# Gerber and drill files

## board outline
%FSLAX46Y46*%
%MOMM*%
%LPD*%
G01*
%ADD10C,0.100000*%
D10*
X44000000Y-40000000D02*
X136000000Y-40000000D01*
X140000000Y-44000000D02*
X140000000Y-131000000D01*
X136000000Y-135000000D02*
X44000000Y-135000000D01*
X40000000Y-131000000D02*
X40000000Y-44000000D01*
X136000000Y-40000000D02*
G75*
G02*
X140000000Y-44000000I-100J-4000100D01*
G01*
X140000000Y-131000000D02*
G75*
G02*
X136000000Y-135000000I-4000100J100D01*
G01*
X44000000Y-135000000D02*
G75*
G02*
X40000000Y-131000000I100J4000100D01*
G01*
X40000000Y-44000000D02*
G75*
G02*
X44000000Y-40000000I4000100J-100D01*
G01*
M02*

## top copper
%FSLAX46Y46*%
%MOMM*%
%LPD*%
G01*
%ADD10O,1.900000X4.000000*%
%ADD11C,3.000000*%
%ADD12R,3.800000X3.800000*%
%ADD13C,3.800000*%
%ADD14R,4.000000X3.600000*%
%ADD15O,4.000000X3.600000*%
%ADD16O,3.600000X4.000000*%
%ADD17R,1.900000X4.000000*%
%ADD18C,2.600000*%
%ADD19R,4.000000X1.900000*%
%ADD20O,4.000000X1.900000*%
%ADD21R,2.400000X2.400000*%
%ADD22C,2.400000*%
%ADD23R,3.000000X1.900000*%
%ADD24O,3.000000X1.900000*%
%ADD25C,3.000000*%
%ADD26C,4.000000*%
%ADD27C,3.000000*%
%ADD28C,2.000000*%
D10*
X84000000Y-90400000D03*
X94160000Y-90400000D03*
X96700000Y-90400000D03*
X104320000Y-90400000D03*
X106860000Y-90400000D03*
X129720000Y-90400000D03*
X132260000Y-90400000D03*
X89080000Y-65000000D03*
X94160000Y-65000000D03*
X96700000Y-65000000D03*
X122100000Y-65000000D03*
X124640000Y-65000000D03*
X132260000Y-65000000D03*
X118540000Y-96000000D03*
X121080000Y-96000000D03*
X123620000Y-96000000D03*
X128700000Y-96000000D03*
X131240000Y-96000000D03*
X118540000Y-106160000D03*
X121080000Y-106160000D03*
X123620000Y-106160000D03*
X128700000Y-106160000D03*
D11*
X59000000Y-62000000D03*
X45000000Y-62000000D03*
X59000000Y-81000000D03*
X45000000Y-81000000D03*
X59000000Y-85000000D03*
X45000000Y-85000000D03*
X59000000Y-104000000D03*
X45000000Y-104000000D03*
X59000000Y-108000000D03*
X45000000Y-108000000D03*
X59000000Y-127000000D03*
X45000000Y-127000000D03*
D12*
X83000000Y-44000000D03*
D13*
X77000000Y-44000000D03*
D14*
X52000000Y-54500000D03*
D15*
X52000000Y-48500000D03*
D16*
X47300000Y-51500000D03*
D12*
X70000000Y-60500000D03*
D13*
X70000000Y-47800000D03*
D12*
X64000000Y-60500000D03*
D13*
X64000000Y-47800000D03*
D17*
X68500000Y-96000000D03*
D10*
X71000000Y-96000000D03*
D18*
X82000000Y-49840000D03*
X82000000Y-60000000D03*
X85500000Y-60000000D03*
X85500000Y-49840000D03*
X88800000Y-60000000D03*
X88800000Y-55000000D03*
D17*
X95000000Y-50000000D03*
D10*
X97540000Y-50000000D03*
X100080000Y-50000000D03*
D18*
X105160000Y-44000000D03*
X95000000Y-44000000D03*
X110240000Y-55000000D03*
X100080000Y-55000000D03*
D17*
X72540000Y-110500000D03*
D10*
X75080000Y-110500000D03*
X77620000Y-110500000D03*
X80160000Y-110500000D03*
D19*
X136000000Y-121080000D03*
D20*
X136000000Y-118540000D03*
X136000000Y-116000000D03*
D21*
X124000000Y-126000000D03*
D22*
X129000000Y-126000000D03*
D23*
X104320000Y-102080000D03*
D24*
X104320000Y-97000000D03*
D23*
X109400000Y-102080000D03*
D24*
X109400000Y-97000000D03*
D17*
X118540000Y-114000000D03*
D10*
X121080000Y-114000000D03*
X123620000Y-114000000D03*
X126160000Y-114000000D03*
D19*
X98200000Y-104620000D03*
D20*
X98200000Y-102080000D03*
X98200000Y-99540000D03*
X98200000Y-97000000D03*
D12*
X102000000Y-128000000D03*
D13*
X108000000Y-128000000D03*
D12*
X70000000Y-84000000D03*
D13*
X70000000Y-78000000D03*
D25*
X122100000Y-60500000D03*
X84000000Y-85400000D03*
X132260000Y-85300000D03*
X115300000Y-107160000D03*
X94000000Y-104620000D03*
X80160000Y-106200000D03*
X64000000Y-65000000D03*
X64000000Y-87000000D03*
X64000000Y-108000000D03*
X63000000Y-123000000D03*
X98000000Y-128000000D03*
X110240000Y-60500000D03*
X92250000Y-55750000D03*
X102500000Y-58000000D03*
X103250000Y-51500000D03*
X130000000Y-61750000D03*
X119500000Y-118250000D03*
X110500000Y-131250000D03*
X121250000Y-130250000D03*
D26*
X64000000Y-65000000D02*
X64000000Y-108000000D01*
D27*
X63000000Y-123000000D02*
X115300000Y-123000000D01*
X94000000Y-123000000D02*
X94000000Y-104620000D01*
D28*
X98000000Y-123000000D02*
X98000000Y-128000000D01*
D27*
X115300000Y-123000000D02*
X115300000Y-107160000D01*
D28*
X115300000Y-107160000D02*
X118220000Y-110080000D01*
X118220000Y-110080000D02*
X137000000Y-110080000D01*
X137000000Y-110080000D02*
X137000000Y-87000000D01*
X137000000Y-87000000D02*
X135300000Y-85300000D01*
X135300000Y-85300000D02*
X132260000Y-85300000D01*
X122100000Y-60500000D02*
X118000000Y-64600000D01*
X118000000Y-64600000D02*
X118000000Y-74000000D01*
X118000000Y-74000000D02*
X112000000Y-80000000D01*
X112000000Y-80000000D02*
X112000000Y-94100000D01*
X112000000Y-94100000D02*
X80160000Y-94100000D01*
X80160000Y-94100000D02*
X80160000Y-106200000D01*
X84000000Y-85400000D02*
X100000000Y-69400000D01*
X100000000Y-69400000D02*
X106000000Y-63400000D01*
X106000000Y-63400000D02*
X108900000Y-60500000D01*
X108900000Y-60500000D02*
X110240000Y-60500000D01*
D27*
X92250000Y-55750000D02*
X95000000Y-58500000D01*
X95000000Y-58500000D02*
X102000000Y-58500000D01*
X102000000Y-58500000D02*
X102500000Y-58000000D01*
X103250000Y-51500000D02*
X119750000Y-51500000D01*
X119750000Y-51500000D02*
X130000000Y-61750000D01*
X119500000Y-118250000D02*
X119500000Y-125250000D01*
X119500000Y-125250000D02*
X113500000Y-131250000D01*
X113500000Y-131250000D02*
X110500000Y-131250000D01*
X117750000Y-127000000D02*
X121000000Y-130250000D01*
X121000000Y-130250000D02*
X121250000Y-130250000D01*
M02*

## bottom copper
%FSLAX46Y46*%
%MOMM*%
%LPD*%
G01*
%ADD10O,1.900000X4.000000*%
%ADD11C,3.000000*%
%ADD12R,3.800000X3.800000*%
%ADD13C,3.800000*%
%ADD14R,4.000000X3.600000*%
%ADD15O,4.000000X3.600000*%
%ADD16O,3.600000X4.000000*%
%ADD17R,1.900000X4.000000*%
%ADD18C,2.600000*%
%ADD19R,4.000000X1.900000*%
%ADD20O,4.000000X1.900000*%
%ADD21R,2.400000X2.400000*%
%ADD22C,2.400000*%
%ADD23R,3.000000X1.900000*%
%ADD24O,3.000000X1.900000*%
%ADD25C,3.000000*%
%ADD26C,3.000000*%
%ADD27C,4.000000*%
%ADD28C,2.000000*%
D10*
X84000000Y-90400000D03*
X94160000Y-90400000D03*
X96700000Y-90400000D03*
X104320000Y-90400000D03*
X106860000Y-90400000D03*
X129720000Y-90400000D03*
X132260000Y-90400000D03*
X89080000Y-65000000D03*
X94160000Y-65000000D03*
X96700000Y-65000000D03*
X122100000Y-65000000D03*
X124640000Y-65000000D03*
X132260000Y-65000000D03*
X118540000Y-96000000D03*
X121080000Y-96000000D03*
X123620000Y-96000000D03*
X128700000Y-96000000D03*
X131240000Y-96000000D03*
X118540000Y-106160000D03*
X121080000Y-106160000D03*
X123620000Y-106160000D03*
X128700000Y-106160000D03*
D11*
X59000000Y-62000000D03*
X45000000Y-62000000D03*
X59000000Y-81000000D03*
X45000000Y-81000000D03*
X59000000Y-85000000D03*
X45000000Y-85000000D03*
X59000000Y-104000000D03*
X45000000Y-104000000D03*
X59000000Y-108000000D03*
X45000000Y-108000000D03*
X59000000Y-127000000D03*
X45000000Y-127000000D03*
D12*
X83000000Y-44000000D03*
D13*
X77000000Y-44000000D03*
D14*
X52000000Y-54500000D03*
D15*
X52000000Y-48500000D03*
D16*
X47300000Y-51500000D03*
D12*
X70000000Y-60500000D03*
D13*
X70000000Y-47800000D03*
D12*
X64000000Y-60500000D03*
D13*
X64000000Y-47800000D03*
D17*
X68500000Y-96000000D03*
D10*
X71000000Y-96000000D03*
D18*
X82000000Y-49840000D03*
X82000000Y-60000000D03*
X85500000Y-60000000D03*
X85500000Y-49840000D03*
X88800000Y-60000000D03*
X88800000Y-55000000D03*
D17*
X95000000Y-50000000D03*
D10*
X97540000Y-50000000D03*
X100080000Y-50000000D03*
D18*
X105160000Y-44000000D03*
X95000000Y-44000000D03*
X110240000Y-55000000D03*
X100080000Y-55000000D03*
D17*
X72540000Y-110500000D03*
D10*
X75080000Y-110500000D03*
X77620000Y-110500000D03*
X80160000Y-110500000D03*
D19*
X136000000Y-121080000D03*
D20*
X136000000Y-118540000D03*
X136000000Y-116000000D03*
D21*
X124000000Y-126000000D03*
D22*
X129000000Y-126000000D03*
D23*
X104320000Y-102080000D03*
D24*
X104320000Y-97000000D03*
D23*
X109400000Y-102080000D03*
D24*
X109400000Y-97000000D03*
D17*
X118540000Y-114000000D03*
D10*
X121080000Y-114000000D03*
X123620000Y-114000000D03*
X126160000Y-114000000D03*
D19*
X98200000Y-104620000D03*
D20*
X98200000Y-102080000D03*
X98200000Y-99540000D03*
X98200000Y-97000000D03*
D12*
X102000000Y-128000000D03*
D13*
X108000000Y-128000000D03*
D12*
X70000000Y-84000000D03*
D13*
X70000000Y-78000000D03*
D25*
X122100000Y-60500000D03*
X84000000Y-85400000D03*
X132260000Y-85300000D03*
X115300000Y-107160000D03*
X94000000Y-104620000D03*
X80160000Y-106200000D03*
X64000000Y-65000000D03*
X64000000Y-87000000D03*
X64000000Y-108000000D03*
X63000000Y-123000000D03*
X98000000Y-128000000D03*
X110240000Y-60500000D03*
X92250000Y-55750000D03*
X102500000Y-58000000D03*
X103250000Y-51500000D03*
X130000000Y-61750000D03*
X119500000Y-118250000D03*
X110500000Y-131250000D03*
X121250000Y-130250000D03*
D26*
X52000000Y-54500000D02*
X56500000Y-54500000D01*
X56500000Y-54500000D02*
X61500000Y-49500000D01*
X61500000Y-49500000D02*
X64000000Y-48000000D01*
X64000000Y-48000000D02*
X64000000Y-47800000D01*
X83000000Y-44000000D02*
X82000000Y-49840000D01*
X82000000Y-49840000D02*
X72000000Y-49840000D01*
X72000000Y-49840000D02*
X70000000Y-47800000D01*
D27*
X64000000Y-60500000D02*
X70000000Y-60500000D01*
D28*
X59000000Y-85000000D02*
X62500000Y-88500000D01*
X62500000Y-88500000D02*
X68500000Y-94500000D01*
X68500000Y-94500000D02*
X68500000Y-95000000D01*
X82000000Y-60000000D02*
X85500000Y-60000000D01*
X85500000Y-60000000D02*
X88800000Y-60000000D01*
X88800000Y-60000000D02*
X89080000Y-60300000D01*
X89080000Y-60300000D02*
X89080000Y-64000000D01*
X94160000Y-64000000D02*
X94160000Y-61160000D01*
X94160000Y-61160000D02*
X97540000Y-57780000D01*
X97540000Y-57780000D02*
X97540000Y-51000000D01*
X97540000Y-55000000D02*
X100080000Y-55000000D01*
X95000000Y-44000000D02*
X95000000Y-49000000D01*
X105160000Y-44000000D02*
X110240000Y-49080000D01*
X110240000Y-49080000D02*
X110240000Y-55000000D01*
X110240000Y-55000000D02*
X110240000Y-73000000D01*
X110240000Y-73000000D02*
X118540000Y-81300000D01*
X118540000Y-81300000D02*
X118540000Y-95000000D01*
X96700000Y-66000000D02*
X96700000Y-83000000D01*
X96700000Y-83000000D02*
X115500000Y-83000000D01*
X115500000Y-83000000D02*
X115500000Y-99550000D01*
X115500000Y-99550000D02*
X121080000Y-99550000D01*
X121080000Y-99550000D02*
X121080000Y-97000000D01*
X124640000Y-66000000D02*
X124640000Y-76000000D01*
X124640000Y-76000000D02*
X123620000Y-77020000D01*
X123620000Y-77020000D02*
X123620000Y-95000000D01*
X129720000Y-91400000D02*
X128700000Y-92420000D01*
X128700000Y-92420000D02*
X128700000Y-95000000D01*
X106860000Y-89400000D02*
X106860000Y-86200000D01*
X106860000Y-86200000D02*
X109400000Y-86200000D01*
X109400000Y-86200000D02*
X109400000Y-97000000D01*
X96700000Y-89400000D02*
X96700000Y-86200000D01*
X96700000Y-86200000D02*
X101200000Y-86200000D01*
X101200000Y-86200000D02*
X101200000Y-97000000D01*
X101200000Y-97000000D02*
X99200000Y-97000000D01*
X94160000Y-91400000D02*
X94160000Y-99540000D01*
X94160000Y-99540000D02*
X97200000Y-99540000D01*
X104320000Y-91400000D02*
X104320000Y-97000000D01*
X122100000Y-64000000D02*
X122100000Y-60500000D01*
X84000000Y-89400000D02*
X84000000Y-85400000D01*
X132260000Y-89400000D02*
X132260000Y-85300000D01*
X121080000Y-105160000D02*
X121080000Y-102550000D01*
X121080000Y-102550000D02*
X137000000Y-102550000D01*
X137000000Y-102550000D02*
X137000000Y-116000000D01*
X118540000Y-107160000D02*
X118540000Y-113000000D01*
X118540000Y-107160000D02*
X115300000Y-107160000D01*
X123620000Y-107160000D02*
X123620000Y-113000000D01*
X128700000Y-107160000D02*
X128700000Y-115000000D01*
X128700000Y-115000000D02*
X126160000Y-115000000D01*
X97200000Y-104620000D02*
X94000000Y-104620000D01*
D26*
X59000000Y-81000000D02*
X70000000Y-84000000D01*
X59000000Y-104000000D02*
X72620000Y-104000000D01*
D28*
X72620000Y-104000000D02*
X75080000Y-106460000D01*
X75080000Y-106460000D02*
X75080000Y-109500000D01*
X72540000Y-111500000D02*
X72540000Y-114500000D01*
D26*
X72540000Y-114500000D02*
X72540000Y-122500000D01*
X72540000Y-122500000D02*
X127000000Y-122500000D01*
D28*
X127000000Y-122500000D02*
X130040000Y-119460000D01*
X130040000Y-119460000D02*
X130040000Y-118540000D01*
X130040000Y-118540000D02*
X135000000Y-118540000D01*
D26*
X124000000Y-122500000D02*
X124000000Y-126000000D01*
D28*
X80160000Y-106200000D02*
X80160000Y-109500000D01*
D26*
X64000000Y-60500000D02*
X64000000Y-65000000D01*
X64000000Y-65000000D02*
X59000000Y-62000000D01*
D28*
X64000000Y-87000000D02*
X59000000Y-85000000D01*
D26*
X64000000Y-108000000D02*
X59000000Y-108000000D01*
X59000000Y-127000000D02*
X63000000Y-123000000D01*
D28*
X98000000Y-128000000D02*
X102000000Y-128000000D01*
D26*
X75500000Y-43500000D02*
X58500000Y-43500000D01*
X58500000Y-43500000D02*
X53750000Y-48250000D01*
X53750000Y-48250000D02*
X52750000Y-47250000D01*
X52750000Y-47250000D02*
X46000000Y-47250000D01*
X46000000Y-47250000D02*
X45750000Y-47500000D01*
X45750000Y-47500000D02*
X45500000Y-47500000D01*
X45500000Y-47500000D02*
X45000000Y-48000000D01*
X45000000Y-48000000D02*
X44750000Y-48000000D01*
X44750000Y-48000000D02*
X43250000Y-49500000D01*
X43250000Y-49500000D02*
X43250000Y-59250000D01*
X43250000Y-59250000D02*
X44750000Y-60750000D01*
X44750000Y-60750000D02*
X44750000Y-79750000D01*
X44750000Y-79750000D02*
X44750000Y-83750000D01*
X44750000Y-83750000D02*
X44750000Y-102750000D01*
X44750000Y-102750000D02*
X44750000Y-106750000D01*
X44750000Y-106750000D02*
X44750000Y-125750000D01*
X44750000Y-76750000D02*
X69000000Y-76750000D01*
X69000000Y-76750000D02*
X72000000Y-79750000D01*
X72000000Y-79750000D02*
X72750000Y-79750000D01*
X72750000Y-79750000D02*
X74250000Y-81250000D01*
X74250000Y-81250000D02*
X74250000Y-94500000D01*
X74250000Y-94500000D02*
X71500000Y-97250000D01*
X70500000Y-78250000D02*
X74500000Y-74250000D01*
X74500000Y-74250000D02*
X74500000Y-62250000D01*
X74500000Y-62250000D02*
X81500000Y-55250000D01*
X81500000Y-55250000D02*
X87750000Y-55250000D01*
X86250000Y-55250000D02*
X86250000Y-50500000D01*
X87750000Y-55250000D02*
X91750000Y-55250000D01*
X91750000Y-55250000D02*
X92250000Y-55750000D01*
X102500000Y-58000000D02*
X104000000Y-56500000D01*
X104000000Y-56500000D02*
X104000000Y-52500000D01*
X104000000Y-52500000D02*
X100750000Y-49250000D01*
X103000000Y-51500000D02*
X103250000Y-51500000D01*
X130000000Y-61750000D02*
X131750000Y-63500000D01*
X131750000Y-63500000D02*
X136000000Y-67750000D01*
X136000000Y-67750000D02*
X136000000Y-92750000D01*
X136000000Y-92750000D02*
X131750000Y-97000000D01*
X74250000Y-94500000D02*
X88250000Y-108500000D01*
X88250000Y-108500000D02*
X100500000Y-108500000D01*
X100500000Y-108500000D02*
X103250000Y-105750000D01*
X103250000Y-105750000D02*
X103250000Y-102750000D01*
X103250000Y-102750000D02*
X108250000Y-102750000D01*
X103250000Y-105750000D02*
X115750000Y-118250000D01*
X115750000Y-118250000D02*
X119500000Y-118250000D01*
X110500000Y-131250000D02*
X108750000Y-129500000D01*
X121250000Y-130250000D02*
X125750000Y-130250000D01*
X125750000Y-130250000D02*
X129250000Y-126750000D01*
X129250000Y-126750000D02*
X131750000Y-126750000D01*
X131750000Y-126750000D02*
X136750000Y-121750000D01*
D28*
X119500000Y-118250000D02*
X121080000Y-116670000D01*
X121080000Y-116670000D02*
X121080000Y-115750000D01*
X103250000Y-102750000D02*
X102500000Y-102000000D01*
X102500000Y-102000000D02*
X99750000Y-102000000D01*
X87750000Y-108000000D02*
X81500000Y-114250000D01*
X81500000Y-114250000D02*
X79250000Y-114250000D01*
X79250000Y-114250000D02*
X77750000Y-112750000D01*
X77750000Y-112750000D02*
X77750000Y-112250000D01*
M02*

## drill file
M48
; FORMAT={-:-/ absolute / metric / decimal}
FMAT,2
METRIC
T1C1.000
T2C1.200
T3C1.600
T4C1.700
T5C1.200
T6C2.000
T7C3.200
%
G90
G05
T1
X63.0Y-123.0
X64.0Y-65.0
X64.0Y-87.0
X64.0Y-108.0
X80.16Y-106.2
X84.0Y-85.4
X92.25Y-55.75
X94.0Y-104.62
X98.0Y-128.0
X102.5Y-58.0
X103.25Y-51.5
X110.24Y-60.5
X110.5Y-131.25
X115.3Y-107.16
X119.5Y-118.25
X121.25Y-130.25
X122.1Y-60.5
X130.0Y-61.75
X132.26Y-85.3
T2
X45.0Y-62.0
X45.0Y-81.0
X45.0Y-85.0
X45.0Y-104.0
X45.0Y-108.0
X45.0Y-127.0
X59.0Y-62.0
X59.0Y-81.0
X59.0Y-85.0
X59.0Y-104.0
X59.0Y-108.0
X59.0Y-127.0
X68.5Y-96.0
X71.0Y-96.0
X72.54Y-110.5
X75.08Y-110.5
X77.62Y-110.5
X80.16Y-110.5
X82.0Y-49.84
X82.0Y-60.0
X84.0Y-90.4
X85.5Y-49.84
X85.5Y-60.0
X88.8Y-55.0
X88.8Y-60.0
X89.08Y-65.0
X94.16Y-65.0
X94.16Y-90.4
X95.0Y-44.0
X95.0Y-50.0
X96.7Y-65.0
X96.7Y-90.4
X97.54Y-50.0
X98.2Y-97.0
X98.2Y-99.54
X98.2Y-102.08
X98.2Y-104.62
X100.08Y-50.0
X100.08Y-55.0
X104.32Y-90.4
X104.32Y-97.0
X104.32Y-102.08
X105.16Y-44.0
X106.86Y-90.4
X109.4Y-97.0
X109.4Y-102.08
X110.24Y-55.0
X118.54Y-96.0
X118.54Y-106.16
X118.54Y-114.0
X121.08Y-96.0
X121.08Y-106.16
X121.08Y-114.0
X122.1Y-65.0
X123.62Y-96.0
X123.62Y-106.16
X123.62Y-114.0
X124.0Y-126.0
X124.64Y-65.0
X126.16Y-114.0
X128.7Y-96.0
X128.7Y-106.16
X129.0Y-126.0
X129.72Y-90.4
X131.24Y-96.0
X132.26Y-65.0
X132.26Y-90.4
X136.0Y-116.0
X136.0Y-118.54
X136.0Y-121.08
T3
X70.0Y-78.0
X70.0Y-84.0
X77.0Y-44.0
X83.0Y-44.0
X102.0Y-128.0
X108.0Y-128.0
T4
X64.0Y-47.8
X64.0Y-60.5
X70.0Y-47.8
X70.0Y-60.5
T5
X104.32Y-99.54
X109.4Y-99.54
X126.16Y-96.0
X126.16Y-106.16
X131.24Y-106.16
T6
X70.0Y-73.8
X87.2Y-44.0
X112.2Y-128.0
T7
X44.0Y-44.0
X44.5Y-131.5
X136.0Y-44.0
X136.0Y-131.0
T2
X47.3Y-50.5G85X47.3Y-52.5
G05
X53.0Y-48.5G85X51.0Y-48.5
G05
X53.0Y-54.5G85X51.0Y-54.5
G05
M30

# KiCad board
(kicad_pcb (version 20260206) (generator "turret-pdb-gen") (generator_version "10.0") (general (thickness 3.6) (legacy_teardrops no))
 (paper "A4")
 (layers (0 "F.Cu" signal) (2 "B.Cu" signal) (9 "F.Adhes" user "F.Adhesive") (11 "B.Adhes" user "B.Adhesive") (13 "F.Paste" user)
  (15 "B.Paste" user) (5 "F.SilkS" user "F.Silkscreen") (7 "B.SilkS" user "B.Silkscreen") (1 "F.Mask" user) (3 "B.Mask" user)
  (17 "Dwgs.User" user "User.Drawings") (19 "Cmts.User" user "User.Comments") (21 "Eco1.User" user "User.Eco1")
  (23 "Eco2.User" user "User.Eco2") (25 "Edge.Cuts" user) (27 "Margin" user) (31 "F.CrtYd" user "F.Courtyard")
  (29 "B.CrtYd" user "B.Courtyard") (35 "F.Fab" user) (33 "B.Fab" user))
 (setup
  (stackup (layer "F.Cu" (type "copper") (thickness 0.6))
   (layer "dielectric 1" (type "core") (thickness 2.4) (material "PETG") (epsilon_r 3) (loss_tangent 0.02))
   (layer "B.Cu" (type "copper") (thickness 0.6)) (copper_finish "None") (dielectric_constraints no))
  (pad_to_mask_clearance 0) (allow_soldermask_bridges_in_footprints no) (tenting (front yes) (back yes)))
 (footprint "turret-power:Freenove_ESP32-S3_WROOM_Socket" (layer "F.Cu") (at 84 90.4)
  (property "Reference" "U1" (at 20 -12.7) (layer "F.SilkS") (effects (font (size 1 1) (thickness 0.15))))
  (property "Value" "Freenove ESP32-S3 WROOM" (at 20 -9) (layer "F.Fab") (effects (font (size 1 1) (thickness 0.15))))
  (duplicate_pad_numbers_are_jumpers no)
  (pad "L1" thru_hole oval (at 0 0) (size 1.9 4) (drill 1.2) (layers "*.Cu" "B.Mask") (zone_connect 0) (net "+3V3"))
  (pad "L5" thru_hole oval (at 10.16 0) (size 1.9 4) (drill 1.2) (layers "*.Cu" "B.Mask") (zone_connect 0) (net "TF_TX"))
  (pad "L6" thru_hole oval (at 12.7 0) (size 1.9 4) (drill 1.2) (layers "*.Cu" "B.Mask") (zone_connect 0) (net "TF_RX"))
  (pad "L9" thru_hole oval (at 20.32 0) (size 1.9 4) (drill 1.2) (layers "*.Cu" "B.Mask") (zone_connect 0) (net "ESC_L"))
  (pad "L10" thru_hole oval (at 22.86 0) (size 1.9 4) (drill 1.2) (layers "*.Cu" "B.Mask") (zone_connect 0) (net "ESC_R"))
  (pad "L19" thru_hole oval (at 45.72 0) (size 1.9 4) (drill 1.2) (layers "*.Cu" "B.Mask") (zone_connect 0) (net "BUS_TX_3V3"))
  (pad "L20" thru_hole oval (at 48.26 0) (size 1.9 4) (drill 1.2) (layers "*.Cu" "B.Mask") (zone_connect 0) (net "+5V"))
  (pad "R3" thru_hole oval (at 5.08 -25.4) (size 1.9 4) (drill 1.2) (layers "*.Cu" "B.Mask") (zone_connect 0) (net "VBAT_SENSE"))
  (pad "R5" thru_hole oval (at 10.16 -25.4) (size 1.9 4) (drill 1.2) (layers "*.Cu" "B.Mask") (zone_connect 0) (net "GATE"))
  (pad "R6" thru_hole oval (at 12.7 -25.4) (size 1.9 4) (drill 1.2) (layers "*.Cu" "B.Mask") (zone_connect 0) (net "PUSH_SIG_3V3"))
  (pad "R16" thru_hole oval (at 38.1 -25.4) (size 1.9 4) (drill 1.2) (layers "*.Cu" "B.Mask") (zone_connect 0) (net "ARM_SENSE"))
  (pad "R17" thru_hole oval (at 40.64 -25.4) (size 1.9 4) (drill 1.2) (layers "*.Cu" "B.Mask") (zone_connect 0) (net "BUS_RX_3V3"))
  (pad "R20" thru_hole oval (at 48.26 -25.4) (size 1.9 4) (drill 1.2) (layers "*.Cu" "B.Mask") (zone_connect 0) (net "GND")))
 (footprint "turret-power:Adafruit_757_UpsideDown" (layer "F.Cu") (at 118.54 96)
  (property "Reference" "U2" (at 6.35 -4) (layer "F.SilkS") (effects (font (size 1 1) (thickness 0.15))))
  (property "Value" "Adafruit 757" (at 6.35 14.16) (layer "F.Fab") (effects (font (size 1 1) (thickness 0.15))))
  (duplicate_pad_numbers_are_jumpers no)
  (pad "LV" thru_hole oval (at 0 0) (size 1.9 4) (drill 1.2) (layers "*.Cu" "B.Mask") (zone_connect 0) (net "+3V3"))
  (pad "A1" thru_hole oval (at 2.54 0) (size 1.9 4) (drill 1.2) (layers "*.Cu" "B.Mask") (zone_connect 0) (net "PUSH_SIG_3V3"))
  (pad "A2" thru_hole oval (at 5.08 0) (size 1.9 4) (drill 1.2) (layers "*.Cu" "B.Mask") (zone_connect 0) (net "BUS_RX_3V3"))
  (pad "" np_thru_hole circle (at 7.62 0) (size 1.2 1.2) (drill 1.2) (layers "*.Cu" "*.Mask"))
  (pad "A4" thru_hole oval (at 10.16 0) (size 1.9 4) (drill 1.2) (layers "*.Cu" "B.Mask") (zone_connect 0) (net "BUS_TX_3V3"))
  (pad "GND_LV" thru_hole oval (at 12.7 0) (size 1.9 4) (drill 1.2) (layers "*.Cu" "B.Mask") (zone_connect 0) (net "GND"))
  (pad "HV" thru_hole oval (at 0 10.16) (size 1.9 4) (drill 1.2) (layers "*.Cu" "B.Mask") (zone_connect 0) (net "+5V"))
  (pad "B1" thru_hole oval (at 2.54 10.16) (size 1.9 4) (drill 1.2) (layers "*.Cu" "B.Mask") (zone_connect 0) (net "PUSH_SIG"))
  (pad "B2" thru_hole oval (at 5.08 10.16) (size 1.9 4) (drill 1.2) (layers "*.Cu" "B.Mask") (zone_connect 0) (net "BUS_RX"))
  (pad "" np_thru_hole circle (at 7.62 10.16) (size 1.2 1.2) (drill 1.2) (layers "*.Cu" "*.Mask"))
  (pad "B4" thru_hole oval (at 10.16 10.16) (size 1.9 4) (drill 1.2) (layers "*.Cu" "B.Mask") (zone_connect 0) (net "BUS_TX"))
  (pad "" np_thru_hole circle (at 12.7 10.16) (size 1.2 1.2) (drill 1.2) (layers "*.Cu" "*.Mask")))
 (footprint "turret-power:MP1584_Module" (layer "F.Cu") (at 59 62 270)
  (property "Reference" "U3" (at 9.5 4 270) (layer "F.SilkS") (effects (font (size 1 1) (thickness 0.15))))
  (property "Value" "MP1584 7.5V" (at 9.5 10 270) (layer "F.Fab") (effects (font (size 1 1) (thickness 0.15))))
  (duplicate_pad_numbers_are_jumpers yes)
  (pad "VIN" thru_hole circle (at 0 0 270) (size 3 3) (drill 1.2) (layers "*.Cu" "*.Mask") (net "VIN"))
  (pad "GND" thru_hole circle (at 0 14 270) (size 3 3) (drill 1.2) (layers "*.Cu" "*.Mask") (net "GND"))
  (pad "VOUT" thru_hole circle (at 19 0 270) (size 3 3) (drill 1.2) (layers "*.Cu" "*.Mask") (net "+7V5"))
  (pad "GND" thru_hole circle (at 19 14 270) (size 3 3) (drill 1.2) (layers "*.Cu" "*.Mask") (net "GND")))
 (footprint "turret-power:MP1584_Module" (layer "F.Cu") (at 59 85 270)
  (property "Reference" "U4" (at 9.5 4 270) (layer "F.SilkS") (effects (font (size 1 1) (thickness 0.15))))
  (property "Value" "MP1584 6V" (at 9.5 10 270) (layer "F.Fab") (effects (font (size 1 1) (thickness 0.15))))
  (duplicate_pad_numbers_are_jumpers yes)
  (pad "VIN" thru_hole circle (at 0 0 270) (size 3 3) (drill 1.2) (layers "*.Cu" "*.Mask") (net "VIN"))
  (pad "GND" thru_hole circle (at 0 14 270) (size 3 3) (drill 1.2) (layers "*.Cu" "*.Mask") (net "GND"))
  (pad "VOUT" thru_hole circle (at 19 0 270) (size 3 3) (drill 1.2) (layers "*.Cu" "*.Mask") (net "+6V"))
  (pad "GND" thru_hole circle (at 19 14 270) (size 3 3) (drill 1.2) (layers "*.Cu" "*.Mask") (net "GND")))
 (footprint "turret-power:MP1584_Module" (layer "F.Cu") (at 59 108 270)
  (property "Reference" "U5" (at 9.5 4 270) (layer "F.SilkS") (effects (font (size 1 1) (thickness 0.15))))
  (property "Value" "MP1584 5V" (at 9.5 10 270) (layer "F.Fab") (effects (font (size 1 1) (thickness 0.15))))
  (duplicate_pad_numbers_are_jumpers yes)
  (pad "VIN" thru_hole circle (at 0 0 270) (size 3 3) (drill 1.2) (layers "*.Cu" "*.Mask") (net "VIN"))
  (pad "GND" thru_hole circle (at 0 14 270) (size 3 3) (drill 1.2) (layers "*.Cu" "*.Mask") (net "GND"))
  (pad "VOUT" thru_hole circle (at 19 0 270) (size 3 3) (drill 1.2) (layers "*.Cu" "*.Mask") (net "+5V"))
  (pad "GND" thru_hole circle (at 19 14 270) (size 3 3) (drill 1.2) (layers "*.Cu" "*.Mask") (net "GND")))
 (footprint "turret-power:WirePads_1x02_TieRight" (layer "F.Cu") (at 83 44 180)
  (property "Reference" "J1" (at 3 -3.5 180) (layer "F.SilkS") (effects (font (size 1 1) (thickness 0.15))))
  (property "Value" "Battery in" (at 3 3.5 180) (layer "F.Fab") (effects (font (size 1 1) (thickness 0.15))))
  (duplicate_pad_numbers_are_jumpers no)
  (pad "1" thru_hole rect (at 0 0 180) (size 3.8 3.8) (drill 1.6) (layers "*.Cu" "*.Mask") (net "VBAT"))
  (pad "2" thru_hole circle (at 6 0 180) (size 3.8 3.8) (drill 1.6) (layers "*.Cu" "*.Mask") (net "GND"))
  (pad "" np_thru_hole circle (at -4.2 0) (size 2 2) (drill 2) (layers "*.Cu" "*.Mask")))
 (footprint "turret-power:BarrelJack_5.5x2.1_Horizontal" (layer "F.Cu") (at 52 54.5 270)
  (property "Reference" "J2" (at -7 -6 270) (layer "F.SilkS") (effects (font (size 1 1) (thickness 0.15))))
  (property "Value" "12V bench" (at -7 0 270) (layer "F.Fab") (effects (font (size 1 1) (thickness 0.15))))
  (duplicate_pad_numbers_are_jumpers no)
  (pad "1" thru_hole rect (at 0 0 270) (size 3.6 4) (drill oval 1.2 3.2) (layers "*.Cu" "B.Mask") (zone_connect 0) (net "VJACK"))
  (pad "2" thru_hole oval (at -6 0 270) (size 3.6 4) (drill oval 1.2 3.2) (layers "*.Cu" "B.Mask") (zone_connect 0) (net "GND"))
  (pad "3" thru_hole oval (at -3 4.7 270) (size 4 3.6) (drill oval 3.2 1.2) (layers "*.Cu" "B.Mask") (zone_connect 0)
   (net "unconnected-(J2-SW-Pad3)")))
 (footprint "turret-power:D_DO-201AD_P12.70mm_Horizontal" (layer "F.Cu") (at 70 60.5 90)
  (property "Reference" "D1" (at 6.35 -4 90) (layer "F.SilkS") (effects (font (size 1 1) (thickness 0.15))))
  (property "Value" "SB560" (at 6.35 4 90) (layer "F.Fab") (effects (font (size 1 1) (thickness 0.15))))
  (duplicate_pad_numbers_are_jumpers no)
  (pad "1" thru_hole rect (at 0 0 90) (size 3.8 3.8) (drill 1.7) (layers "*.Cu" "*.Mask") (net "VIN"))
  (pad "2" thru_hole circle (at 12.7 0 90) (size 3.8 3.8) (drill 1.7) (layers "*.Cu" "*.Mask") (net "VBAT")))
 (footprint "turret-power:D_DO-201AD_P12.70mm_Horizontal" (layer "F.Cu") (at 64 60.5 90)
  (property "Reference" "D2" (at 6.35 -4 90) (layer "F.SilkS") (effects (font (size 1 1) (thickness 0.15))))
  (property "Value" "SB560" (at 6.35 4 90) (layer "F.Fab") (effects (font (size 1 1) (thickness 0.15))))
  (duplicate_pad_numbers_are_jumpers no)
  (pad "1" thru_hole rect (at 0 0 90) (size 3.8 3.8) (drill 1.7) (layers "*.Cu" "*.Mask") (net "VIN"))
  (pad "2" thru_hole circle (at 12.7 0 90) (size 3.8 3.8) (drill 1.7) (layers "*.Cu" "*.Mask") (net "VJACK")))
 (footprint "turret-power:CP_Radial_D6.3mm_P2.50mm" (layer "F.Cu") (at 68.5 96)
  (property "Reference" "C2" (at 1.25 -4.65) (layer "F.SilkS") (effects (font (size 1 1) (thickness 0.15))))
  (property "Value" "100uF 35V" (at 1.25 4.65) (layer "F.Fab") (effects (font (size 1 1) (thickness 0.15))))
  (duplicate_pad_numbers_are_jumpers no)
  (pad "1" thru_hole rect (at 0 0) (size 1.9 4) (drill 1.2) (layers "*.Cu" "B.Mask") (zone_connect 0) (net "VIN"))
  (pad "2" thru_hole oval (at 2.5 0) (size 1.9 4) (drill 1.2) (layers "*.Cu" "B.Mask") (zone_connect 0) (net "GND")))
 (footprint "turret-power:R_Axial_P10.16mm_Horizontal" (layer "F.Cu") (at 82 49.84 270)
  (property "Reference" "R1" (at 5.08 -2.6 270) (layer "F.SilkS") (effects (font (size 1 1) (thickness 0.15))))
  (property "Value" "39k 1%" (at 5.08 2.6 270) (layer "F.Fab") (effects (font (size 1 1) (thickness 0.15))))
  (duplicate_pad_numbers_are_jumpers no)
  (pad "1" thru_hole circle (at 0 0 270) (size 2.6 2.6) (drill 1.2) (layers "*.Cu" "*.Mask") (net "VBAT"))
  (pad "2" thru_hole circle (at 10.16 0 270) (size 2.6 2.6) (drill 1.2) (layers "*.Cu" "*.Mask") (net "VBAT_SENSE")))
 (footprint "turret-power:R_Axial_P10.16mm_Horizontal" (layer "F.Cu") (at 85.5 60 90)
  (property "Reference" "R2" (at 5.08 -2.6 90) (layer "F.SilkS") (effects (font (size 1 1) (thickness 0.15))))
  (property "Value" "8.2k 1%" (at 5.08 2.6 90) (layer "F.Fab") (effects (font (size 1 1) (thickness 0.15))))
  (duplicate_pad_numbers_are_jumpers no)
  (pad "1" thru_hole circle (at 0 0 90) (size 2.6 2.6) (drill 1.2) (layers "*.Cu" "*.Mask") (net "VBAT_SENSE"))
  (pad "2" thru_hole circle (at 10.16 0 90) (size 2.6 2.6) (drill 1.2) (layers "*.Cu" "*.Mask") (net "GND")))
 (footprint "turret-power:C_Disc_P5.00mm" (layer "F.Cu") (at 88.8 60 90)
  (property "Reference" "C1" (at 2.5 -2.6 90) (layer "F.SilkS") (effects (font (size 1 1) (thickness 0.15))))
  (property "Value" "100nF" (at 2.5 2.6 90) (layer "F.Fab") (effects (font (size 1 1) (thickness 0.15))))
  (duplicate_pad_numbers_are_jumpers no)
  (pad "1" thru_hole circle (at 0 0 90) (size 2.6 2.6) (drill 1.2) (layers "*.Cu" "*.Mask") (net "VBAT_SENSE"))
  (pad "2" thru_hole circle (at 5 0 90) (size 2.6 2.6) (drill 1.2) (layers "*.Cu" "*.Mask") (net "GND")))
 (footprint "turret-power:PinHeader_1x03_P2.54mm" (layer "F.Cu") (at 95 50)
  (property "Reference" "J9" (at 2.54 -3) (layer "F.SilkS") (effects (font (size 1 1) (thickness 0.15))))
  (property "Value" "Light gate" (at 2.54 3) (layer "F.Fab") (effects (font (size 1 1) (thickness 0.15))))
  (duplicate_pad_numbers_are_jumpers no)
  (pad "1" thru_hole rect (at 0 0) (size 1.9 4) (drill 1.2) (layers "*.Cu" "B.Mask") (zone_connect 0) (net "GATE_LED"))
  (pad "2" thru_hole oval (at 2.54 0) (size 1.9 4) (drill 1.2) (layers "*.Cu" "B.Mask") (zone_connect 0) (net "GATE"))
  (pad "3" thru_hole oval (at 5.08 0) (size 1.9 4) (drill 1.2) (layers "*.Cu" "B.Mask") (zone_connect 0) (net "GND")))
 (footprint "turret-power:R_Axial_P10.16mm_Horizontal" (layer "F.Cu") (at 105.16 44 180)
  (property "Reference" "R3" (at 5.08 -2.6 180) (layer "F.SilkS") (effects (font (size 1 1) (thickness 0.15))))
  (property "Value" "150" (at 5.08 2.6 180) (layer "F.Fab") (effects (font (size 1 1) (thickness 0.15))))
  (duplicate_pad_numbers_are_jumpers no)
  (pad "1" thru_hole circle (at 0 0 180) (size 2.6 2.6) (drill 1.2) (layers "*.Cu" "*.Mask") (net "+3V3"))
  (pad "2" thru_hole circle (at 10.16 0 180) (size 2.6 2.6) (drill 1.2) (layers "*.Cu" "*.Mask") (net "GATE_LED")))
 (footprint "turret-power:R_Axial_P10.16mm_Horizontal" (layer "F.Cu") (at 110.24 55 180)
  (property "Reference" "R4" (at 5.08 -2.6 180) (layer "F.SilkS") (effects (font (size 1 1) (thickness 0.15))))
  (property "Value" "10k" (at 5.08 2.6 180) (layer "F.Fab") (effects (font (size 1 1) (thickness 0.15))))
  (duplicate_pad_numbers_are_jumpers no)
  (pad "1" thru_hole circle (at 0 0 180) (size 2.6 2.6) (drill 1.2) (layers "*.Cu" "*.Mask") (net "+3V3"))
  (pad "2" thru_hole circle (at 10.16 0 180) (size 2.6 2.6) (drill 1.2) (layers "*.Cu" "*.Mask") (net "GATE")))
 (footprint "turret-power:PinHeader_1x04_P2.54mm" (layer "F.Cu") (at 72.54 110.5)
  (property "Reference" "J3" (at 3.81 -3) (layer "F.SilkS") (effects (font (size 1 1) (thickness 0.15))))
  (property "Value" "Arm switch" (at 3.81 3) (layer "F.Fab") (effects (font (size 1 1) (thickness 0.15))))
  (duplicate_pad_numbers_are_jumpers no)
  (pad "1" thru_hole rect (at 0 0) (size 1.9 4) (drill 1.2) (layers "*.Cu" "B.Mask") (zone_connect 0) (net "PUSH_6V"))
  (pad "2" thru_hole oval (at 2.54 0) (size 1.9 4) (drill 1.2) (layers "*.Cu" "B.Mask") (zone_connect 0) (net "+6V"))
  (pad "3" thru_hole oval (at 5.08 0) (size 1.9 4) (drill 1.2) (layers "*.Cu" "B.Mask") (zone_connect 0) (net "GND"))
  (pad "4" thru_hole oval (at 7.62 0) (size 1.9 4) (drill 1.2) (layers "*.Cu" "B.Mask") (zone_connect 0) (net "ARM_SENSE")))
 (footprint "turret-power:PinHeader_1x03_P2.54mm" (layer "F.Cu") (at 136 121.08 90)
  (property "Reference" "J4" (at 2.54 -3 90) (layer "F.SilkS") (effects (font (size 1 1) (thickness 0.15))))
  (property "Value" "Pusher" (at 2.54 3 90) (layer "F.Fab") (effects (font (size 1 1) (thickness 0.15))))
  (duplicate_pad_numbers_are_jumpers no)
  (pad "1" thru_hole rect (at 0 0 90) (size 1.9 4) (drill 1.2) (layers "*.Cu" "B.Mask") (zone_connect 0) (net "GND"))
  (pad "2" thru_hole oval (at 2.54 0 90) (size 1.9 4) (drill 1.2) (layers "*.Cu" "B.Mask") (zone_connect 0) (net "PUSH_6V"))
  (pad "3" thru_hole oval (at 5.08 0 90) (size 1.9 4) (drill 1.2) (layers "*.Cu" "B.Mask") (zone_connect 0) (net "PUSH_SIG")))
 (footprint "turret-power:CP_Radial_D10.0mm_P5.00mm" (layer "F.Cu") (at 124 126)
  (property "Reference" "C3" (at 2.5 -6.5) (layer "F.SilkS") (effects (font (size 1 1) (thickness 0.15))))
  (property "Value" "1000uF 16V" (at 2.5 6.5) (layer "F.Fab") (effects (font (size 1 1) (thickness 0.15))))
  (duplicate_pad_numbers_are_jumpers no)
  (pad "1" thru_hole rect (at 0 0) (size 2.4 2.4) (drill 1.2) (layers "*.Cu" "B.Mask") (zone_connect 0) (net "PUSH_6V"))
  (pad "2" thru_hole circle (at 5 0) (size 2.4 2.4) (drill 1.2) (layers "*.Cu" "B.Mask") (zone_connect 0) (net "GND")))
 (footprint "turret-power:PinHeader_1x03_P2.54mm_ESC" (layer "F.Cu") (at 104.32 102.08 90)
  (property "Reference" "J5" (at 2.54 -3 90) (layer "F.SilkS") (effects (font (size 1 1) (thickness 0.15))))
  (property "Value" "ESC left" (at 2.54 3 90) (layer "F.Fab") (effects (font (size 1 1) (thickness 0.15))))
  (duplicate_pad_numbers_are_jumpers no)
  (pad "1" thru_hole rect (at 0 0 90) (size 1.9 3) (drill 1.2) (layers "*.Cu" "B.Mask") (zone_connect 0) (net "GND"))
  (pad "" np_thru_hole circle (at 2.54 0) (size 1.2 1.2) (drill 1.2) (layers "*.Cu" "*.Mask"))
  (pad "3" thru_hole oval (at 5.08 0 90) (size 1.9 3) (drill 1.2) (layers "*.Cu" "B.Mask") (zone_connect 0) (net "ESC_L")))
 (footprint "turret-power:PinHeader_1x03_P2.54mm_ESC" (layer "F.Cu") (at 109.4 102.08 90)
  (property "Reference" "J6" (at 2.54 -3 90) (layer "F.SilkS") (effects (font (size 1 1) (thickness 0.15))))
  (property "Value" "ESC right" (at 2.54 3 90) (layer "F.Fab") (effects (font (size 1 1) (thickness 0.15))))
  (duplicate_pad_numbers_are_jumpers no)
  (pad "1" thru_hole rect (at 0 0 90) (size 1.9 3) (drill 1.2) (layers "*.Cu" "B.Mask") (zone_connect 0) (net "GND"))
  (pad "" np_thru_hole circle (at 2.54 0) (size 1.2 1.2) (drill 1.2) (layers "*.Cu" "*.Mask"))
  (pad "3" thru_hole oval (at 5.08 0 90) (size 1.9 3) (drill 1.2) (layers "*.Cu" "B.Mask") (zone_connect 0) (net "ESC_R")))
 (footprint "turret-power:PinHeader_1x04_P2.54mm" (layer "F.Cu") (at 118.54 114)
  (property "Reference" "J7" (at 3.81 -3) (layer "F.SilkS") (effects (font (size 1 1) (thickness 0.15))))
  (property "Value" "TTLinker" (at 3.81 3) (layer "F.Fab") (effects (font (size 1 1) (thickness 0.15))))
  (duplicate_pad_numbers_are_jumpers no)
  (pad "1" thru_hole rect (at 0 0) (size 1.9 4) (drill 1.2) (layers "*.Cu" "B.Mask") (zone_connect 0) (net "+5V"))
  (pad "2" thru_hole oval (at 2.54 0) (size 1.9 4) (drill 1.2) (layers "*.Cu" "B.Mask") (zone_connect 0) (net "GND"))
  (pad "3" thru_hole oval (at 5.08 0) (size 1.9 4) (drill 1.2) (layers "*.Cu" "B.Mask") (zone_connect 0) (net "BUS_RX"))
  (pad "4" thru_hole oval (at 7.62 0) (size 1.9 4) (drill 1.2) (layers "*.Cu" "B.Mask") (zone_connect 0) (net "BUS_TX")))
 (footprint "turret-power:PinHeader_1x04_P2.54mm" (layer "F.Cu") (at 98.2 104.62 90)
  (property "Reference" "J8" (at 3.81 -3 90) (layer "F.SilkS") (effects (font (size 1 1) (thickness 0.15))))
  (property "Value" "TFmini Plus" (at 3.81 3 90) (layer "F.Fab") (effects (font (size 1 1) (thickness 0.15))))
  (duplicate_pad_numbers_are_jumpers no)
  (pad "1" thru_hole rect (at 0 0 90) (size 1.9 4) (drill 1.2) (layers "*.Cu" "B.Mask") (zone_connect 0) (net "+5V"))
  (pad "2" thru_hole oval (at 2.54 0 90) (size 1.9 4) (drill 1.2) (layers "*.Cu" "B.Mask") (zone_connect 0) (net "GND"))
  (pad "3" thru_hole oval (at 5.08 0 90) (size 1.9 4) (drill 1.2) (layers "*.Cu" "B.Mask") (zone_connect 0) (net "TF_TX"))
  (pad "4" thru_hole oval (at 7.62 0 90) (size 1.9 4) (drill 1.2) (layers "*.Cu" "B.Mask") (zone_connect 0) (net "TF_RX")))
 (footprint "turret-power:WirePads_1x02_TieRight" (layer "F.Cu") (at 102 128)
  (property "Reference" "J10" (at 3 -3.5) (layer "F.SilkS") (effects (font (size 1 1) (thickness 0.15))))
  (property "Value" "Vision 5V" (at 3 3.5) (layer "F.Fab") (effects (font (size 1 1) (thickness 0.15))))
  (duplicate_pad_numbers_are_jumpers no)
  (pad "1" thru_hole rect (at 0 0) (size 3.8 3.8) (drill 1.6) (layers "*.Cu" "*.Mask") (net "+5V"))
  (pad "2" thru_hole circle (at 6 0) (size 3.8 3.8) (drill 1.6) (layers "*.Cu" "*.Mask") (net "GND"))
  (pad "" np_thru_hole circle (at 10.2 0) (size 2 2) (drill 2) (layers "*.Cu" "*.Mask")))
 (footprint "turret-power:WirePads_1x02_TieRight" (layer "F.Cu") (at 70 84 90)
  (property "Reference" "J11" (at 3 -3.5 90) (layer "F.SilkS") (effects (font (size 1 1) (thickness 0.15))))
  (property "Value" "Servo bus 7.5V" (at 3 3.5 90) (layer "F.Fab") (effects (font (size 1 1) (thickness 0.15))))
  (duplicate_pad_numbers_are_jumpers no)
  (pad "1" thru_hole rect (at 0 0 90) (size 3.8 3.8) (drill 1.6) (layers "*.Cu" "*.Mask") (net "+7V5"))
  (pad "2" thru_hole circle (at 6 0 90) (size 3.8 3.8) (drill 1.6) (layers "*.Cu" "*.Mask") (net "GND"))
  (pad "" np_thru_hole circle (at 10.2 0) (size 2 2) (drill 2) (layers "*.Cu" "*.Mask")))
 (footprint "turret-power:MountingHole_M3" (layer "F.Cu") (at 44 44)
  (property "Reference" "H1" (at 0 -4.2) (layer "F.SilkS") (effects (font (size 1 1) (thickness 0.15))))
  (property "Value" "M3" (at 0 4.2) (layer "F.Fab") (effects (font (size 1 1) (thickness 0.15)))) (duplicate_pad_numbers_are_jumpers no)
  (pad "" np_thru_hole circle (at 0 0) (size 3.2 3.2) (drill 3.2) (layers "*.Cu" "*.Mask")))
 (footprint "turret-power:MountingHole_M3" (layer "F.Cu") (at 136 44)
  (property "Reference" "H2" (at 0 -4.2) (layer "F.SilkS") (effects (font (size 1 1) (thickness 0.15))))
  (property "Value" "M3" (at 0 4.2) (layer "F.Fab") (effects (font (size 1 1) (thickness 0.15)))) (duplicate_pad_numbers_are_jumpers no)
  (pad "" np_thru_hole circle (at 0 0) (size 3.2 3.2) (drill 3.2) (layers "*.Cu" "*.Mask")))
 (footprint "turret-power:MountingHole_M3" (layer "F.Cu") (at 44.5 131.5)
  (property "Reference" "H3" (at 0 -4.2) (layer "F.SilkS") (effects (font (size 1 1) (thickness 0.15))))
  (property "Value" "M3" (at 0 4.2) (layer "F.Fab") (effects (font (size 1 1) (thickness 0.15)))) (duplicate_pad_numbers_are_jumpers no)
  (pad "" np_thru_hole circle (at 0 0) (size 3.2 3.2) (drill 3.2) (layers "*.Cu" "*.Mask")))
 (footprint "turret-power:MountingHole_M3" (layer "F.Cu") (at 136 131)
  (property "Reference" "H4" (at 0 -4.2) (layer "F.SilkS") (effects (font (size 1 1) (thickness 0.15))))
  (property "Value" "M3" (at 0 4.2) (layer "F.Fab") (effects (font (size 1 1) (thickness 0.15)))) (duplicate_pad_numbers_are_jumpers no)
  (pad "" np_thru_hole circle (at 0 0) (size 3.2 3.2) (drill 3.2) (layers "*.Cu" "*.Mask")))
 (gr_line (start 44 40) (end 136 40) (stroke (width 0.1) (type default)) (layer "Edge.Cuts"))
 (gr_line (start 140 44) (end 140 131) (stroke (width 0.1) (type default)) (layer "Edge.Cuts"))
 (gr_line (start 136 135) (end 44 135) (stroke (width 0.1) (type default)) (layer "Edge.Cuts"))
 (gr_line (start 40 131) (end 40 44) (stroke (width 0.1) (type default)) (layer "Edge.Cuts"))
 (gr_arc (start 136 40) (mid 138.8284 41.1716) (end 140 44) (stroke (width 0.1) (type default)) (layer "Edge.Cuts"))
 (gr_arc (start 140 131) (mid 138.8284 133.8284) (end 136 135) (stroke (width 0.1) (type default)) (layer "Edge.Cuts"))
 (gr_arc (start 44 135) (mid 41.1716 133.8284) (end 40 131) (stroke (width 0.1) (type default)) (layer "Edge.Cuts"))
 (gr_arc (start 40 44) (mid 41.1716 41.1716) (end 44 40) (stroke (width 0.1) (type default)) (layer "Edge.Cuts"))
 (segment (start 52 54.5) (end 56.5 54.5) (width 3) (layer "B.Cu") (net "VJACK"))
 (segment (start 56.5 54.5) (end 61.5 49.5) (width 3) (layer "B.Cu") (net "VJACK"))
 (segment (start 61.5 49.5) (end 64 48) (width 3) (layer "B.Cu") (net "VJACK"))
 (segment (start 64 48) (end 64 47.8) (width 3) (layer "B.Cu") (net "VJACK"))
 (segment (start 83 44) (end 82 49.84) (width 3) (layer "B.Cu") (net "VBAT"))
 (segment (start 82 49.84) (end 72 49.84) (width 3) (layer "B.Cu") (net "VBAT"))
 (segment (start 72 49.84) (end 70 47.8) (width 3) (layer "B.Cu") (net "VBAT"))
 (segment (start 64 60.5) (end 70 60.5) (width 4) (layer "B.Cu") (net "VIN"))
 (segment (start 59 85) (end 62.5 88.5) (width 2) (layer "B.Cu") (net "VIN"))
 (segment (start 62.5 88.5) (end 68.5 94.5) (width 2) (layer "B.Cu") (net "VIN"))
 (segment (start 68.5 94.5) (end 68.5 95) (width 2) (layer "B.Cu") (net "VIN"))
 (segment (start 82 60) (end 85.5 60) (width 2) (layer "B.Cu") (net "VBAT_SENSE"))
 (segment (start 85.5 60) (end 88.8 60) (width 2) (layer "B.Cu") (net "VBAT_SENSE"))
 (segment (start 88.8 60) (end 89.08 60.3) (width 2) (layer "B.Cu") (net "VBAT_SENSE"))
 (segment (start 89.08 60.3) (end 89.08 64) (width 2) (layer "B.Cu") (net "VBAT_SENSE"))
 (segment (start 94.16 64) (end 94.16 61.16) (width 2) (layer "B.Cu") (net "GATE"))
 (segment (start 94.16 61.16) (end 97.54 57.78) (width 2) (layer "B.Cu") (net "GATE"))
 (segment (start 97.54 57.78) (end 97.54 51) (width 2) (layer "B.Cu") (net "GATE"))
 (segment (start 97.54 55) (end 100.08 55) (width 2) (layer "B.Cu") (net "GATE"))
 (segment (start 95 44) (end 95 49) (width 2) (layer "B.Cu") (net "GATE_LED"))
 (segment (start 105.16 44) (end 110.24 49.08) (width 2) (layer "B.Cu") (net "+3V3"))
 (segment (start 110.24 49.08) (end 110.24 55) (width 2) (layer "B.Cu") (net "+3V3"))
 (segment (start 110.24 55) (end 110.24 73) (width 2) (layer "B.Cu") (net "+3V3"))
 (segment (start 110.24 73) (end 118.54 81.3) (width 2) (layer "B.Cu") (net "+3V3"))
 (segment (start 118.54 81.3) (end 118.54 95) (width 2) (layer "B.Cu") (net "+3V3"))
 (segment (start 96.7 66) (end 96.7 83) (width 2) (layer "B.Cu") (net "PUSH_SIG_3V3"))
 (segment (start 96.7 83) (end 115.5 83) (width 2) (layer "B.Cu") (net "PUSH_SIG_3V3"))
 (segment (start 115.5 83) (end 115.5 99.55) (width 2) (layer "B.Cu") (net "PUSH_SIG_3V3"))
 (segment (start 115.5 99.55) (end 121.08 99.55) (width 2) (layer "B.Cu") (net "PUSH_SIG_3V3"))
 (segment (start 121.08 99.55) (end 121.08 97) (width 2) (layer "B.Cu") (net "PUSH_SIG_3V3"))
 (segment (start 124.64 66) (end 124.64 76) (width 2) (layer "B.Cu") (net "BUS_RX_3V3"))
 (segment (start 124.64 76) (end 123.62 77.02) (width 2) (layer "B.Cu") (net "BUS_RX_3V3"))
 (segment (start 123.62 77.02) (end 123.62 95) (width 2) (layer "B.Cu") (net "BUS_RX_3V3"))
 (segment (start 129.72 91.4) (end 128.7 92.42) (width 2) (layer "B.Cu") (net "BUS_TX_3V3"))
 (segment (start 128.7 92.42) (end 128.7 95) (width 2) (layer "B.Cu") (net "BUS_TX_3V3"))
 (segment (start 106.86 89.4) (end 106.86 86.2) (width 2) (layer "B.Cu") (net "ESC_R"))
 (segment (start 106.86 86.2) (end 109.4 86.2) (width 2) (layer "B.Cu") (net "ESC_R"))
 (segment (start 109.4 86.2) (end 109.4 97) (width 2) (layer "B.Cu") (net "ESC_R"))
 (segment (start 96.7 89.4) (end 96.7 86.2) (width 2) (layer "B.Cu") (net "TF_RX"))
 (segment (start 96.7 86.2) (end 101.2 86.2) (width 2) (layer "B.Cu") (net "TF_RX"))
 (segment (start 101.2 86.2) (end 101.2 97) (width 2) (layer "B.Cu") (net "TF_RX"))
 (segment (start 101.2 97) (end 99.2 97) (width 2) (layer "B.Cu") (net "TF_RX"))
 (segment (start 94.16 91.4) (end 94.16 99.54) (width 2) (layer "B.Cu") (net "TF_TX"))
 (segment (start 94.16 99.54) (end 97.2 99.54) (width 2) (layer "B.Cu") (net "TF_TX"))
 (segment (start 104.32 91.4) (end 104.32 97) (width 2) (layer "B.Cu") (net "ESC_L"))
 (segment (start 122.1 64) (end 122.1 60.5) (width 2) (layer "B.Cu") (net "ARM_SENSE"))
 (segment (start 84 89.4) (end 84 85.4) (width 2) (layer "B.Cu") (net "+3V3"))
 (segment (start 132.26 89.4) (end 132.26 85.3) (width 2) (layer "B.Cu") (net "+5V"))
 (segment (start 121.08 105.16) (end 121.08 102.55) (width 2) (layer "B.Cu") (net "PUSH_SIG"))
 (segment (start 121.08 102.55) (end 137 102.55) (width 2) (layer "B.Cu") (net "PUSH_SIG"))
 (segment (start 137 102.55) (end 137 116) (width 2) (layer "B.Cu") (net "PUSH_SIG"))
 (segment (start 118.54 107.16) (end 118.54 113) (width 2) (layer "B.Cu") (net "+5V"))
 (segment (start 118.54 107.16) (end 115.3 107.16) (width 2) (layer "B.Cu") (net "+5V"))
 (segment (start 123.62 107.16) (end 123.62 113) (width 2) (layer "B.Cu") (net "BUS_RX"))
 (segment (start 128.7 107.16) (end 128.7 115) (width 2) (layer "B.Cu") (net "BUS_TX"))
 (segment (start 128.7 115) (end 126.16 115) (width 2) (layer "B.Cu") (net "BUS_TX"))
 (segment (start 97.2 104.62) (end 94 104.62) (width 2) (layer "B.Cu") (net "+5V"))
 (segment (start 59 81) (end 70 84) (width 3) (layer "B.Cu") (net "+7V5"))
 (segment (start 59 104) (end 72.62 104) (width 3) (layer "B.Cu") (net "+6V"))
 (segment (start 72.62 104) (end 75.08 106.46) (width 2) (layer "B.Cu") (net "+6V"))
 (segment (start 75.08 106.46) (end 75.08 109.5) (width 2) (layer "B.Cu") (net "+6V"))
 (segment (start 72.54 111.5) (end 72.54 114.5) (width 2) (layer "B.Cu") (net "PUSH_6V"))
 (segment (start 72.54 114.5) (end 72.54 122.5) (width 3) (layer "B.Cu") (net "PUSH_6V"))
 (segment (start 72.54 122.5) (end 127 122.5) (width 3) (layer "B.Cu") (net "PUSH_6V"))
 (segment (start 127 122.5) (end 130.04 119.46) (width 2) (layer "B.Cu") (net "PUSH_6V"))
 (segment (start 130.04 119.46) (end 130.04 118.54) (width 2) (layer "B.Cu") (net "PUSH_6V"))
 (segment (start 130.04 118.54) (end 135 118.54) (width 2) (layer "B.Cu") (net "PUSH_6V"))
 (segment (start 124 122.5) (end 124 126) (width 3) (layer "B.Cu") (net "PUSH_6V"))
 (segment (start 80.16 106.2) (end 80.16 109.5) (width 2) (layer "B.Cu") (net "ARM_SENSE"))
 (segment (start 64 65) (end 64 108) (width 4) (layer "F.Cu") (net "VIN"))
 (segment (start 64 60.5) (end 64 65) (width 3) (layer "B.Cu") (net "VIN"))
 (segment (start 64 65) (end 59 62) (width 3) (layer "B.Cu") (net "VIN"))
 (segment (start 64 87) (end 59 85) (width 2) (layer "B.Cu") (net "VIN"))
 (segment (start 64 108) (end 59 108) (width 3) (layer "B.Cu") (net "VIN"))
 (segment (start 59 127) (end 63 123) (width 3) (layer "B.Cu") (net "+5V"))
 (segment (start 63 123) (end 115.3 123) (width 3) (layer "F.Cu") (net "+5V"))
 (segment (start 94 123) (end 94 104.62) (width 3) (layer "F.Cu") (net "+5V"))
 (segment (start 98 123) (end 98 128) (width 2) (layer "F.Cu") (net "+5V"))
 (segment (start 98 128) (end 102 128) (width 2) (layer "B.Cu") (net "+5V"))
 (segment (start 115.3 123) (end 115.3 107.16) (width 3) (layer "F.Cu") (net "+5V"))
 (segment (start 115.3 107.16) (end 118.22 110.08) (width 2) (layer "F.Cu") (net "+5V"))
 (segment (start 118.22 110.08) (end 137 110.08) (width 2) (layer "F.Cu") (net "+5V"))
 (segment (start 137 110.08) (end 137 87) (width 2) (layer "F.Cu") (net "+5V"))
 (segment (start 137 87) (end 135.3 85.3) (width 2) (layer "F.Cu") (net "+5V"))
 (segment (start 135.3 85.3) (end 132.26 85.3) (width 2) (layer "F.Cu") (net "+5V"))
 (segment (start 122.1 60.5) (end 118 64.6) (width 2) (layer "F.Cu") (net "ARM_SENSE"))
 (segment (start 118 64.6) (end 118 74) (width 2) (layer "F.Cu") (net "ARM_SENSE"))
 (segment (start 118 74) (end 112 80) (width 2) (layer "F.Cu") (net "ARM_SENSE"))
 (segment (start 112 80) (end 112 94.1) (width 2) (layer "F.Cu") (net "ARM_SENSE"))
 (segment (start 112 94.1) (end 80.16 94.1) (width 2) (layer "F.Cu") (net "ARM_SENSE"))
 (segment (start 80.16 94.1) (end 80.16 106.2) (width 2) (layer "F.Cu") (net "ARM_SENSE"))
 (segment (start 84 85.4) (end 100 69.4) (width 2) (layer "F.Cu") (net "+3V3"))
 (segment (start 100 69.4) (end 106 63.4) (width 2) (layer "F.Cu") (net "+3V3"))
 (segment (start 106 63.4) (end 108.9 60.5) (width 2) (layer "F.Cu") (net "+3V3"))
 (segment (start 108.9 60.5) (end 110.24 60.5) (width 2) (layer "F.Cu") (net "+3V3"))
 (segment (start 75.5 43.5) (end 58.5 43.5) (width 3) (layer "B.Cu") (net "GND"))
 (segment (start 58.5 43.5) (end 53.75 48.25) (width 3) (layer "B.Cu") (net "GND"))
 (segment (start 53.75 48.25) (end 52.75 47.25) (width 3) (layer "B.Cu") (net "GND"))
 (segment (start 52.75 47.25) (end 46 47.25) (width 3) (layer "B.Cu") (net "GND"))
 (segment (start 46 47.25) (end 45.75 47.5) (width 3) (layer "B.Cu") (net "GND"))
 (segment (start 45.75 47.5) (end 45.5 47.5) (width 3) (layer "B.Cu") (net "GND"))
 (segment (start 45.5 47.5) (end 45 48) (width 3) (layer "B.Cu") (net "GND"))
 (segment (start 45 48) (end 44.75 48) (width 3) (layer "B.Cu") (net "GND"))
 (segment (start 44.75 48) (end 43.25 49.5) (width 3) (layer "B.Cu") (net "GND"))
 (segment (start 43.25 49.5) (end 43.25 59.25) (width 3) (layer "B.Cu") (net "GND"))
 (segment (start 43.25 59.25) (end 44.75 60.75) (width 3) (layer "B.Cu") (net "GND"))
 (segment (start 44.75 60.75) (end 44.75 79.75) (width 3) (layer "B.Cu") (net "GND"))
 (segment (start 44.75 79.75) (end 44.75 83.75) (width 3) (layer "B.Cu") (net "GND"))
 (segment (start 44.75 83.75) (end 44.75 102.75) (width 3) (layer "B.Cu") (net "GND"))
 (segment (start 44.75 102.75) (end 44.75 106.75) (width 3) (layer "B.Cu") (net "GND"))
 (segment (start 44.75 106.75) (end 44.75 125.75) (width 3) (layer "B.Cu") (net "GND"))
 (segment (start 44.75 76.75) (end 69 76.75) (width 3) (layer "B.Cu") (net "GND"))
 (segment (start 69 76.75) (end 72 79.75) (width 3) (layer "B.Cu") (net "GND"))
 (segment (start 72 79.75) (end 72.75 79.75) (width 3) (layer "B.Cu") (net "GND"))
 (segment (start 72.75 79.75) (end 74.25 81.25) (width 3) (layer "B.Cu") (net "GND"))
 (segment (start 74.25 81.25) (end 74.25 94.5) (width 3) (layer "B.Cu") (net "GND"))
 (segment (start 74.25 94.5) (end 71.5 97.25) (width 3) (layer "B.Cu") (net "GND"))
 (segment (start 70.5 78.25) (end 74.5 74.25) (width 3) (layer "B.Cu") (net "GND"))
 (segment (start 74.5 74.25) (end 74.5 62.25) (width 3) (layer "B.Cu") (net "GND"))
 (segment (start 74.5 62.25) (end 81.5 55.25) (width 3) (layer "B.Cu") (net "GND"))
 (segment (start 81.5 55.25) (end 87.75 55.25) (width 3) (layer "B.Cu") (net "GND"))
 (segment (start 86.25 55.25) (end 86.25 50.5) (width 3) (layer "B.Cu") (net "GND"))
 (segment (start 87.75 55.25) (end 91.75 55.25) (width 3) (layer "B.Cu") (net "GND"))
 (segment (start 91.75 55.25) (end 92.25 55.75) (width 3) (layer "B.Cu") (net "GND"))
 (segment (start 92.25 55.75) (end 95 58.5) (width 3) (layer "F.Cu") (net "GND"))
 (segment (start 95 58.5) (end 102 58.5) (width 3) (layer "F.Cu") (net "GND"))
 (segment (start 102 58.5) (end 102.5 58) (width 3) (layer "F.Cu") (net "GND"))
 (segment (start 102.5 58) (end 104 56.5) (width 3) (layer "B.Cu") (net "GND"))
 (segment (start 104 56.5) (end 104 52.5) (width 3) (layer "B.Cu") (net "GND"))
 (segment (start 104 52.5) (end 100.75 49.25) (width 3) (layer "B.Cu") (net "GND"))
 (segment (start 103 51.5) (end 103.25 51.5) (width 3) (layer "B.Cu") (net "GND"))
 (segment (start 103.25 51.5) (end 119.75 51.5) (width 3) (layer "F.Cu") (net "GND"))
 (segment (start 119.75 51.5) (end 130 61.75) (width 3) (layer "F.Cu") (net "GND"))
 (segment (start 130 61.75) (end 131.75 63.5) (width 3) (layer "B.Cu") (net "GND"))
 (segment (start 131.75 63.5) (end 136 67.75) (width 3) (layer "B.Cu") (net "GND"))
 (segment (start 136 67.75) (end 136 92.75) (width 3) (layer "B.Cu") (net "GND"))
 (segment (start 136 92.75) (end 131.75 97) (width 3) (layer "B.Cu") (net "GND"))
 (segment (start 74.25 94.5) (end 88.25 108.5) (width 3) (layer "B.Cu") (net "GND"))
 (segment (start 88.25 108.5) (end 100.5 108.5) (width 3) (layer "B.Cu") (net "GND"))
 (segment (start 100.5 108.5) (end 103.25 105.75) (width 3) (layer "B.Cu") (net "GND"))
 (segment (start 103.25 105.75) (end 103.25 102.75) (width 3) (layer "B.Cu") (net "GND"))
 (segment (start 103.25 102.75) (end 108.25 102.75) (width 3) (layer "B.Cu") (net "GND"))
 (segment (start 103.25 105.75) (end 115.75 118.25) (width 3) (layer "B.Cu") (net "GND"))
 (segment (start 115.75 118.25) (end 119.5 118.25) (width 3) (layer "B.Cu") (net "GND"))
 (segment (start 119.5 118.25) (end 119.5 125.25) (width 3) (layer "F.Cu") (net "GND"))
 (segment (start 119.5 125.25) (end 113.5 131.25) (width 3) (layer "F.Cu") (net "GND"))
 (segment (start 113.5 131.25) (end 110.5 131.25) (width 3) (layer "F.Cu") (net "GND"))
 (segment (start 110.5 131.25) (end 108.75 129.5) (width 3) (layer "B.Cu") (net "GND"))
 (segment (start 117.75 127) (end 121 130.25) (width 3) (layer "F.Cu") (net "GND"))
 (segment (start 121 130.25) (end 121.25 130.25) (width 3) (layer "F.Cu") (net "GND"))
 (segment (start 121.25 130.25) (end 125.75 130.25) (width 3) (layer "B.Cu") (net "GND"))
 (segment (start 125.75 130.25) (end 129.25 126.75) (width 3) (layer "B.Cu") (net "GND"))
 (segment (start 129.25 126.75) (end 131.75 126.75) (width 3) (layer "B.Cu") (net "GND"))
 (segment (start 131.75 126.75) (end 136.75 121.75) (width 3) (layer "B.Cu") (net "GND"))
 (segment (start 119.5 118.25) (end 121.08 116.67) (width 2) (layer "B.Cu") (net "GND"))
 (segment (start 121.08 116.67) (end 121.08 115.75) (width 2) (layer "B.Cu") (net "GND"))
 (segment (start 103.25 102.75) (end 102.5 102) (width 2) (layer "B.Cu") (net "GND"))
 (segment (start 102.5 102) (end 99.75 102) (width 2) (layer "B.Cu") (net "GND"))
 (segment (start 87.75 108) (end 81.5 114.25) (width 2) (layer "B.Cu") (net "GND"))
 (segment (start 81.5 114.25) (end 79.25 114.25) (width 2) (layer "B.Cu") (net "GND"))
 (segment (start 79.25 114.25) (end 77.75 112.75) (width 2) (layer "B.Cu") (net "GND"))
 (segment (start 77.75 112.75) (end 77.75 112.25) (width 2) (layer "B.Cu") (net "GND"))
 (via (at 122.1 60.5) (size 3) (drill 1) (layers "F.Cu" "B.Cu") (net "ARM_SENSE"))
 (via (at 84 85.4) (size 3) (drill 1) (layers "F.Cu" "B.Cu") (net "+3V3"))
 (via (at 132.26 85.3) (size 3) (drill 1) (layers "F.Cu" "B.Cu") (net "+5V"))
 (via (at 115.3 107.16) (size 3) (drill 1) (layers "F.Cu" "B.Cu") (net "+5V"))
 (via (at 94 104.62) (size 3) (drill 1) (layers "F.Cu" "B.Cu") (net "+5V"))
 (via (at 80.16 106.2) (size 3) (drill 1) (layers "F.Cu" "B.Cu") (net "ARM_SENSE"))
 (via (at 64 65) (size 3) (drill 1) (layers "F.Cu" "B.Cu") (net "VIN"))
 (via (at 64 87) (size 3) (drill 1) (layers "F.Cu" "B.Cu") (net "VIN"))
 (via (at 64 108) (size 3) (drill 1) (layers "F.Cu" "B.Cu") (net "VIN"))
 (via (at 63 123) (size 3) (drill 1) (layers "F.Cu" "B.Cu") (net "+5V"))
 (via (at 98 128) (size 3) (drill 1) (layers "F.Cu" "B.Cu") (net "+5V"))
 (via (at 110.24 60.5) (size 3) (drill 1) (layers "F.Cu" "B.Cu") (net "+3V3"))
 (via (at 92.25 55.75) (size 3) (drill 1) (layers "F.Cu" "B.Cu") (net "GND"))
 (via (at 102.5 58) (size 3) (drill 1) (layers "F.Cu" "B.Cu") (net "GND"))
 (via (at 103.25 51.5) (size 3) (drill 1) (layers "F.Cu" "B.Cu") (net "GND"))
 (via (at 130 61.75) (size 3) (drill 1) (layers "F.Cu" "B.Cu") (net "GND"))
 (via (at 119.5 118.25) (size 3) (drill 1) (layers "F.Cu" "B.Cu") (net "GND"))
 (via (at 110.5 131.25) (size 3) (drill 1) (layers "F.Cu" "B.Cu") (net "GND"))
 (via (at 121.25 130.25) (size 3) (drill 1) (layers "F.Cu" "B.Cu") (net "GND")))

